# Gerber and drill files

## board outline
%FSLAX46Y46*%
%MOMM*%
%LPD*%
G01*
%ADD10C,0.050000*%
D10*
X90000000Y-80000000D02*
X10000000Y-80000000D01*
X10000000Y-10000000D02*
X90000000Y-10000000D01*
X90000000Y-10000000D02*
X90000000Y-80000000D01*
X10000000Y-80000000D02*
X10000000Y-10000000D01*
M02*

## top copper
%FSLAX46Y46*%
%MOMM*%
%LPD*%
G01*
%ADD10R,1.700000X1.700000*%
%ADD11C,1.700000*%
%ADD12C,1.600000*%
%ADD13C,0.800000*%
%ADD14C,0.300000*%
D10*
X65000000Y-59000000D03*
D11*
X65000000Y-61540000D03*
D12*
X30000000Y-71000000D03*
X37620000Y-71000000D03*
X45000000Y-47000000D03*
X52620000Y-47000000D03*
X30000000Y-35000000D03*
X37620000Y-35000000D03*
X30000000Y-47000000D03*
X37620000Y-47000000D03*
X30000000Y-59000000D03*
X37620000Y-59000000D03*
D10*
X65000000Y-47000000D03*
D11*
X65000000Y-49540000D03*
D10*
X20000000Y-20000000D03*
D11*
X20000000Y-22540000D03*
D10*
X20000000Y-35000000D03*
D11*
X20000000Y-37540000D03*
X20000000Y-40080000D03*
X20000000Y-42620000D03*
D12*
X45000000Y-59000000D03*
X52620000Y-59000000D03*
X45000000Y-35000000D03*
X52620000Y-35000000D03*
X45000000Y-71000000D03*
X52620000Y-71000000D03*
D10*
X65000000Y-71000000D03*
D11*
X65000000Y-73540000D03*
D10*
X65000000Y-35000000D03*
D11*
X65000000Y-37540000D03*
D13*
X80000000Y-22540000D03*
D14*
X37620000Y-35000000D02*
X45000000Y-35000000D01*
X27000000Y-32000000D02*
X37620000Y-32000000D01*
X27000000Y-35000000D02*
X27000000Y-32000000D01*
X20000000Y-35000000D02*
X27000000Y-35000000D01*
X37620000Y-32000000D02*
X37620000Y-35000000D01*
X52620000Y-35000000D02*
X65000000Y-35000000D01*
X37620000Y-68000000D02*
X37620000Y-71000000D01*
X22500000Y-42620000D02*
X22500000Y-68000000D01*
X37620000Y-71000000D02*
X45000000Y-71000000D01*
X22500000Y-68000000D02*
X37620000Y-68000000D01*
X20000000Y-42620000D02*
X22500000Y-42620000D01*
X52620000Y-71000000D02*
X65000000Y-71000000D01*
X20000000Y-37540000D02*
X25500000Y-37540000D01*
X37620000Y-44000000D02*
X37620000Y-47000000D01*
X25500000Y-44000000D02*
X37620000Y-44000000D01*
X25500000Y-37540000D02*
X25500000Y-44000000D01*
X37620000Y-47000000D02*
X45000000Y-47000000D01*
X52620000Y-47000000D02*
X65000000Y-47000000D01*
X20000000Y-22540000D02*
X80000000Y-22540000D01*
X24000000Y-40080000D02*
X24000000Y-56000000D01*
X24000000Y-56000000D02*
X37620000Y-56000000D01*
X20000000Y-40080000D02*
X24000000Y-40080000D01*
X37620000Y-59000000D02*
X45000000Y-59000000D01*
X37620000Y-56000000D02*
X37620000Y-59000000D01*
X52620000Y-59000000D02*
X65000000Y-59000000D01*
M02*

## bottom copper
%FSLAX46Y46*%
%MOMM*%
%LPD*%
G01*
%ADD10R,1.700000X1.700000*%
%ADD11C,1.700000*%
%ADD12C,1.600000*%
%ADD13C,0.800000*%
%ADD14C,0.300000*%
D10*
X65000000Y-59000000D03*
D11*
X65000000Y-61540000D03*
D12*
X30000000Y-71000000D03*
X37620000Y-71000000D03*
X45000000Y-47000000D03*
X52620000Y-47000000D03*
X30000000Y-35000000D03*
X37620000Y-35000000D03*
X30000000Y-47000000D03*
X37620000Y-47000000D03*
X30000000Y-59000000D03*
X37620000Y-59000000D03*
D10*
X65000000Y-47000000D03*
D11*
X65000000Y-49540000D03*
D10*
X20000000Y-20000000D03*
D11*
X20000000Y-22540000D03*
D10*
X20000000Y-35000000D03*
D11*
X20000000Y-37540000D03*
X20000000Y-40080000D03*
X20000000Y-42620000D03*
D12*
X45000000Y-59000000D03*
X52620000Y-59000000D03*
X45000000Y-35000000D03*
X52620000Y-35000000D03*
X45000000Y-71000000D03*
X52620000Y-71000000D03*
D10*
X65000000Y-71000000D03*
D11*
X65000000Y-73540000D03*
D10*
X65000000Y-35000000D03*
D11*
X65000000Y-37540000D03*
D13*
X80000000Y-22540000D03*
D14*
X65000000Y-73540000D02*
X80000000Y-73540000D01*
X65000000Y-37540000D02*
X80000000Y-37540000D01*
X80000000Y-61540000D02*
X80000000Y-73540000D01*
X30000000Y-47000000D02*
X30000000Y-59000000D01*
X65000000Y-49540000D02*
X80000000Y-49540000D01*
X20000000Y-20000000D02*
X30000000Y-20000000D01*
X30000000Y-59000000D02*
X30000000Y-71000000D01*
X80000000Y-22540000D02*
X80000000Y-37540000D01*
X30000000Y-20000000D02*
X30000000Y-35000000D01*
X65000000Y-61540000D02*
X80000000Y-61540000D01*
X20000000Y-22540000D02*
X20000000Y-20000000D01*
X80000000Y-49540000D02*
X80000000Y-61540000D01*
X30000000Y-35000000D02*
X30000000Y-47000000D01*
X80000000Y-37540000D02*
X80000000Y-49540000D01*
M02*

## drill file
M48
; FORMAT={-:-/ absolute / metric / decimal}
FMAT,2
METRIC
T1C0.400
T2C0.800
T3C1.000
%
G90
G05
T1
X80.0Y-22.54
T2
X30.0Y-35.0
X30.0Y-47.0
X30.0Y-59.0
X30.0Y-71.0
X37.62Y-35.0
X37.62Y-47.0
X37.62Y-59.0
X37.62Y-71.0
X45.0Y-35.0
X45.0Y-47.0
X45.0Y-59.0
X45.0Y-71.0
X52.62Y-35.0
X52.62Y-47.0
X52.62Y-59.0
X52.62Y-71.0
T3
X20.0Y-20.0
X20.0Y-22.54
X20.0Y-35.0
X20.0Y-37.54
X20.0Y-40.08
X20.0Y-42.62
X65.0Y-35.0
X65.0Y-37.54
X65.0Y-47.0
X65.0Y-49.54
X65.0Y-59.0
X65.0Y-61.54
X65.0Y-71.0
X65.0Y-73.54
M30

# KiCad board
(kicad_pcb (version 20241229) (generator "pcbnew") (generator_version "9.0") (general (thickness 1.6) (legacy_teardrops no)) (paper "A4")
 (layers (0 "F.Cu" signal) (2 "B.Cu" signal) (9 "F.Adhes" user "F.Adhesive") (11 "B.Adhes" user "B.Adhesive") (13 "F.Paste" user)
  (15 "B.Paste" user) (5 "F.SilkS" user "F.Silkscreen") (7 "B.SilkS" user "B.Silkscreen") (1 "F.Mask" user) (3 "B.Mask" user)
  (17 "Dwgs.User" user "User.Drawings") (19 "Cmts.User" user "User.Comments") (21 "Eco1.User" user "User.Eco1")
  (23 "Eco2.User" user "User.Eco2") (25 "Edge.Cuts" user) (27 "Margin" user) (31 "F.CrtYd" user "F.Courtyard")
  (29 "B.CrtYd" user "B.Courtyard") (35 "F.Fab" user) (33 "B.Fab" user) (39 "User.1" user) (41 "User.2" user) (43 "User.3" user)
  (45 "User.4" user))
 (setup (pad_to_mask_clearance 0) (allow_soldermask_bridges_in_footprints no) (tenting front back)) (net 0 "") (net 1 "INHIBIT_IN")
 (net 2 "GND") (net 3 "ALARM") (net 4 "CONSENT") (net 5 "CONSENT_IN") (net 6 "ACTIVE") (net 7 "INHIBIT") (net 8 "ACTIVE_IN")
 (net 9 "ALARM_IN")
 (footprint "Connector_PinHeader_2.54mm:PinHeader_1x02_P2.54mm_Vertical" (layer "F.Cu") (at 65 59)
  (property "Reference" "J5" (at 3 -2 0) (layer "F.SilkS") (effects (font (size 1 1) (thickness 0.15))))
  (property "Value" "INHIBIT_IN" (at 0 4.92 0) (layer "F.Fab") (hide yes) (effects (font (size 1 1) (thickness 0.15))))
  (pad "1" thru_hole rect (at 0 0) (size 1.7 1.7) (drill 1) (layers "*.Cu" "*.Mask") (remove_unused_layers no) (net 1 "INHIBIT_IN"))
  (pad "2" thru_hole circle (at 0 2.54) (size 1.7 1.7) (drill 1) (layers "*.Cu" "*.Mask") (remove_unused_layers no) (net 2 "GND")))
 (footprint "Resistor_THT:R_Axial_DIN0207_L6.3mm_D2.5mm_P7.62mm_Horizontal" (layer "F.Cu") (at 30 71)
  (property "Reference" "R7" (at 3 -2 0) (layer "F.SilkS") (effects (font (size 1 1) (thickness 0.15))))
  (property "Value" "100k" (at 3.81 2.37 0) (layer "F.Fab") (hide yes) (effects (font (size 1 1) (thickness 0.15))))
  (pad "1" thru_hole circle (at 0 0) (size 1.6 1.6) (drill 0.8) (layers "*.Cu" "*.Mask") (remove_unused_layers no) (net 2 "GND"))
  (pad "2" thru_hole circle (at 7.62 0) (size 1.6 1.6) (drill 0.8) (layers "*.Cu" "*.Mask") (remove_unused_layers no) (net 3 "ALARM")))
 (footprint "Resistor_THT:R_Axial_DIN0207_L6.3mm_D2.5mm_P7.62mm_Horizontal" (layer "F.Cu") (at 45 47)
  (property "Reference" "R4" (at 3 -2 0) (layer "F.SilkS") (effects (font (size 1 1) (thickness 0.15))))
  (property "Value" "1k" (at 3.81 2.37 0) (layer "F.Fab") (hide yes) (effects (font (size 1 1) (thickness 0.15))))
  (pad "1" thru_hole circle (at 0 0) (size 1.6 1.6) (drill 0.8) (layers "*.Cu" "*.Mask") (remove_unused_layers no) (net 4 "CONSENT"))
  (pad "2" thru_hole circle (at 7.62 0) (size 1.6 1.6) (drill 0.8) (layers "*.Cu" "*.Mask") (remove_unused_layers no) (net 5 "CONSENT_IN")))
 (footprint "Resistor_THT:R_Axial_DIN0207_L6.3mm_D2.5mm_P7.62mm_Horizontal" (layer "F.Cu") (at 30 35)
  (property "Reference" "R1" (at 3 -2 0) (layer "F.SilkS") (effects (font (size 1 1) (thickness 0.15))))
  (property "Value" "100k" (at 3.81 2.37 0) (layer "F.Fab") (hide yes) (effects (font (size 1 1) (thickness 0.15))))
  (pad "1" thru_hole circle (at 0 0) (size 1.6 1.6) (drill 0.8) (layers "*.Cu" "*.Mask") (remove_unused_layers no) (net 2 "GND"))
  (pad "2" thru_hole circle (at 7.62 0) (size 1.6 1.6) (drill 0.8) (layers "*.Cu" "*.Mask") (remove_unused_layers no) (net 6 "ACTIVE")))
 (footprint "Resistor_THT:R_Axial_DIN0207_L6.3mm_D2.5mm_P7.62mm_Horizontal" (layer "F.Cu") (at 30 47)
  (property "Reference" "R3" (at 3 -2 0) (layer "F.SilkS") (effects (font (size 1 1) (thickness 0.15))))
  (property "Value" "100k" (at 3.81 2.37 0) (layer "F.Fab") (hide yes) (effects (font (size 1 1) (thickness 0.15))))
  (pad "1" thru_hole circle (at 0 0) (size 1.6 1.6) (drill 0.8) (layers "*.Cu" "*.Mask") (remove_unused_layers no) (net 2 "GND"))
  (pad "2" thru_hole circle (at 7.62 0) (size 1.6 1.6) (drill 0.8) (layers "*.Cu" "*.Mask") (remove_unused_layers no) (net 4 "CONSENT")))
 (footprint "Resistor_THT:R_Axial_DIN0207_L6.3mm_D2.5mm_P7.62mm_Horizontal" (layer "F.Cu") (at 30 59)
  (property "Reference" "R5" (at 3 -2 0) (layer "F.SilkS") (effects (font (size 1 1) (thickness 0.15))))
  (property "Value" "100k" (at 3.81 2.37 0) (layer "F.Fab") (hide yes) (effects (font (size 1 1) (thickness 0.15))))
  (pad "1" thru_hole circle (at 0 0) (size 1.6 1.6) (drill 0.8) (layers "*.Cu" "*.Mask") (remove_unused_layers no) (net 2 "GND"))
  (pad "2" thru_hole circle (at 7.62 0) (size 1.6 1.6) (drill 0.8) (layers "*.Cu" "*.Mask") (remove_unused_layers no) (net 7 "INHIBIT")))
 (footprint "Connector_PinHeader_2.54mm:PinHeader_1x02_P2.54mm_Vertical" (layer "F.Cu") (at 65 47)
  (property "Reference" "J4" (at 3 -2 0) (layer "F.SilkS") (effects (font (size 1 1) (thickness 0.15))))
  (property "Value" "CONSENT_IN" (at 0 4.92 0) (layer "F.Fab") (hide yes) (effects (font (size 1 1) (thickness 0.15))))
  (pad "1" thru_hole rect (at 0 0) (size 1.7 1.7) (drill 1) (layers "*.Cu" "*.Mask") (remove_unused_layers no) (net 5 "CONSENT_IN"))
  (pad "2" thru_hole circle (at 0 2.54) (size 1.7 1.7) (drill 1) (layers "*.Cu" "*.Mask") (remove_unused_layers no) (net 2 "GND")))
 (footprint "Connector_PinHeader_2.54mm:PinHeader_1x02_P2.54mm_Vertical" (layer "F.Cu") (at 20 20)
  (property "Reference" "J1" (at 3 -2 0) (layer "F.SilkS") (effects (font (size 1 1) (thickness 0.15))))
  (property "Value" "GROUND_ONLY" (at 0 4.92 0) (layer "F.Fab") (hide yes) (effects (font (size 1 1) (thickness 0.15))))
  (pad "1" thru_hole rect (at 0 0) (size 1.7 1.7) (drill 1) (layers "*.Cu" "*.Mask") (remove_unused_layers no) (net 2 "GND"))
  (pad "2" thru_hole circle (at 0 2.54) (size 1.7 1.7) (drill 1) (layers "*.Cu" "*.Mask") (remove_unused_layers no) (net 2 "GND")))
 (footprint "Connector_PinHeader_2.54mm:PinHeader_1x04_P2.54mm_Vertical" (layer "F.Cu") (at 20 35)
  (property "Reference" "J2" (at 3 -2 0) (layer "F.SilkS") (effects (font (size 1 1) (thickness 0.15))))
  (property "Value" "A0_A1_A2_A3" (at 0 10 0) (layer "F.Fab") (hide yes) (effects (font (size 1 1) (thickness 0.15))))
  (pad "1" thru_hole rect (at 0 0) (size 1.7 1.7) (drill 1) (layers "*.Cu" "*.Mask") (remove_unused_layers no) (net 6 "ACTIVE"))
  (pad "2" thru_hole circle (at 0 2.54) (size 1.7 1.7) (drill 1) (layers "*.Cu" "*.Mask") (remove_unused_layers no) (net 4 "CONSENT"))
  (pad "3" thru_hole circle (at 0 5.08) (size 1.7 1.7) (drill 1) (layers "*.Cu" "*.Mask") (remove_unused_layers no) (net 7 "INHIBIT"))
  (pad "4" thru_hole circle (at 0 7.62) (size 1.7 1.7) (drill 1) (layers "*.Cu" "*.Mask") (remove_unused_layers no) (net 3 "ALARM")))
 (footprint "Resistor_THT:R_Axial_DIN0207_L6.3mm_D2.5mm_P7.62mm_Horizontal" (layer "F.Cu") (at 45 59)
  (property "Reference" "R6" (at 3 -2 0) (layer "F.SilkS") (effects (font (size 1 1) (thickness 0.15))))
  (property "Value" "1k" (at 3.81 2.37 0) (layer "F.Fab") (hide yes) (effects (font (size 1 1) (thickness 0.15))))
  (pad "1" thru_hole circle (at 0 0) (size 1.6 1.6) (drill 0.8) (layers "*.Cu" "*.Mask") (remove_unused_layers no) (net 7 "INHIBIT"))
  (pad "2" thru_hole circle (at 7.62 0) (size 1.6 1.6) (drill 0.8) (layers "*.Cu" "*.Mask") (remove_unused_layers no) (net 1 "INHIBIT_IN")))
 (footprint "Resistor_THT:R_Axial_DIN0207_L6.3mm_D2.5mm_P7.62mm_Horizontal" (layer "F.Cu") (at 45 35)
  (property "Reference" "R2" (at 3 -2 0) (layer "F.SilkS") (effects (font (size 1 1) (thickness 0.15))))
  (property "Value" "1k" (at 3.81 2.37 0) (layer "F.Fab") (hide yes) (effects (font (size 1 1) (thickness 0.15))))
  (pad "1" thru_hole circle (at 0 0) (size 1.6 1.6) (drill 0.8) (layers "*.Cu" "*.Mask") (remove_unused_layers no) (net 6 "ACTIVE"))
  (pad "2" thru_hole circle (at 7.62 0) (size 1.6 1.6) (drill 0.8) (layers "*.Cu" "*.Mask") (remove_unused_layers no) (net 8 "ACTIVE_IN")))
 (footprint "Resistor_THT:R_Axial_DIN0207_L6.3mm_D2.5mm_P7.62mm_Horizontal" (layer "F.Cu") (at 45 71)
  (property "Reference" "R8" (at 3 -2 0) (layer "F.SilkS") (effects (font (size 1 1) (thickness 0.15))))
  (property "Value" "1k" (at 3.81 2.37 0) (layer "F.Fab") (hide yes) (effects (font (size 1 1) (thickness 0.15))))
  (pad "1" thru_hole circle (at 0 0) (size 1.6 1.6) (drill 0.8) (layers "*.Cu" "*.Mask") (remove_unused_layers no) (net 3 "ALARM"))
  (pad "2" thru_hole circle (at 7.62 0) (size 1.6 1.6) (drill 0.8) (layers "*.Cu" "*.Mask") (remove_unused_layers no) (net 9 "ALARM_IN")))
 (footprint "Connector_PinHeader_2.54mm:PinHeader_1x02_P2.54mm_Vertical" (layer "F.Cu") (at 65 71)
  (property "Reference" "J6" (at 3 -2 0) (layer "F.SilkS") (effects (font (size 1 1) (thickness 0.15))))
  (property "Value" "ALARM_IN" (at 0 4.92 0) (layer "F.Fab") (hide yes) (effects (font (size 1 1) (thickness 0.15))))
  (pad "1" thru_hole rect (at 0 0) (size 1.7 1.7) (drill 1) (layers "*.Cu" "*.Mask") (remove_unused_layers no) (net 9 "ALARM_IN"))
  (pad "2" thru_hole circle (at 0 2.54) (size 1.7 1.7) (drill 1) (layers "*.Cu" "*.Mask") (remove_unused_layers no) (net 2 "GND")))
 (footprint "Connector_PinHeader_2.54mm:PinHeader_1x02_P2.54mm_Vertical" (layer "F.Cu") (at 65 35)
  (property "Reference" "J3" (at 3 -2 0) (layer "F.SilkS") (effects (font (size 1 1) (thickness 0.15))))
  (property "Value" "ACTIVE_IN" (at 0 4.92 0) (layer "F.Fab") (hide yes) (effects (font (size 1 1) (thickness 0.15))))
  (pad "1" thru_hole rect (at 0 0) (size 1.7 1.7) (drill 1) (layers "*.Cu" "*.Mask") (remove_unused_layers no) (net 8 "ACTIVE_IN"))
  (pad "2" thru_hole circle (at 0 2.54) (size 1.7 1.7) (drill 1) (layers "*.Cu" "*.Mask") (remove_unused_layers no) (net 2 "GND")))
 (gr_line (start 90 80) (end 10 80) (stroke (width 0.05) (type default)) (layer "Edge.Cuts"))
 (gr_line (start 10 10) (end 90 10) (stroke (width 0.05) (type default)) (layer "Edge.Cuts"))
 (gr_line (start 90 10) (end 90 80) (stroke (width 0.05) (type default)) (layer "Edge.Cuts"))
 (gr_line (start 10 80) (end 10 10) (stroke (width 0.05) (type default)) (layer "Edge.Cuts"))
 (segment (start 37.62 35) (end 45 35) (width 0.3) (layer "F.Cu") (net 6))
 (segment (start 27 32) (end 37.62 32) (width 0.3) (layer "F.Cu") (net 6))
 (segment (start 27 35) (end 27 32) (width 0.3) (layer "F.Cu") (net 6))
 (segment (start 20 35) (end 27 35) (width 0.3) (layer "F.Cu") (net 6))
 (segment (start 37.62 32) (end 37.62 35) (width 0.3) (layer "F.Cu") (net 6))
 (segment (start 52.62 35) (end 65 35) (width 0.3) (layer "F.Cu") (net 8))
 (segment (start 37.62 68) (end 37.62 71) (width 0.3) (layer "F.Cu") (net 3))
 (segment (start 22.5 42.62) (end 22.5 68) (width 0.3) (layer "F.Cu") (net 3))
 (segment (start 37.62 71) (end 45 71) (width 0.3) (layer "F.Cu") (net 3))
 (segment (start 22.5 68) (end 37.62 68) (width 0.3) (layer "F.Cu") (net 3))
 (segment (start 20 42.62) (end 22.5 42.62) (width 0.3) (layer "F.Cu") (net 3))
 (segment (start 52.62 71) (end 65 71) (width 0.3) (layer "F.Cu") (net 9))
 (segment (start 20 37.54) (end 25.5 37.54) (width 0.3) (layer "F.Cu") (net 4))
 (segment (start 37.62 44) (end 37.62 47) (width 0.3) (layer "F.Cu") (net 4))
 (segment (start 25.5 44) (end 37.62 44) (width 0.3) (layer "F.Cu") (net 4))
 (segment (start 25.5 37.54) (end 25.5 44) (width 0.3) (layer "F.Cu") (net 4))
 (segment (start 37.62 47) (end 45 47) (width 0.3) (layer "F.Cu") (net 4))
 (segment (start 52.62 47) (end 65 47) (width 0.3) (layer "F.Cu") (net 5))
 (segment (start 20 22.54) (end 80 22.54) (width 0.3) (layer "F.Cu") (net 2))
 (via (at 80 22.54) (size 0.8) (drill 0.4) (layers "F.Cu" "B.Cu") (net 2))
 (segment (start 65 73.54) (end 80 73.54) (width 0.3) (layer "B.Cu") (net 2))
 (segment (start 65 37.54) (end 80 37.54) (width 0.3) (layer "B.Cu") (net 2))
 (segment (start 80 61.54) (end 80 73.54) (width 0.3) (layer "B.Cu") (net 2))
 (segment (start 30 47) (end 30 59) (width 0.3) (layer "B.Cu") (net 2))
 (segment (start 65 49.54) (end 80 49.54) (width 0.3) (layer "B.Cu") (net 2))
 (segment (start 20 20) (end 30 20) (width 0.3) (layer "B.Cu") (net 2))
 (segment (start 30 59) (end 30 71) (width 0.3) (layer "B.Cu") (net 2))
 (segment (start 80 22.54) (end 80 37.54) (width 0.3) (layer "B.Cu") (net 2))
 (segment (start 30 20) (end 30 35) (width 0.3) (layer "B.Cu") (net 2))
 (segment (start 65 61.54) (end 80 61.54) (width 0.3) (layer "B.Cu") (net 2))
 (segment (start 20 22.54) (end 20 20) (width 0.3) (layer "B.Cu") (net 2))
 (segment (start 80 49.54) (end 80 61.54) (width 0.3) (layer "B.Cu") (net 2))
 (segment (start 30 35) (end 30 47) (width 0.3) (layer "B.Cu") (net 2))
 (segment (start 80 37.54) (end 80 49.54) (width 0.3) (layer "B.Cu") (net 2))
 (segment (start 24 40.08) (end 24 56) (width 0.3) (layer "F.Cu") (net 7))
 (segment (start 24 56) (end 37.62 56) (width 0.3) (layer "F.Cu") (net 7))
 (segment (start 20 40.08) (end 24 40.08) (width 0.3) (layer "F.Cu") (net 7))
 (segment (start 37.62 59) (end 45 59) (width 0.3) (layer "F.Cu") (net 7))
 (segment (start 37.62 56) (end 37.62 59) (width 0.3) (layer "F.Cu") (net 7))
 (segment (start 52.62 59) (end 65 59) (width 0.3) (layer "F.Cu") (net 1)))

